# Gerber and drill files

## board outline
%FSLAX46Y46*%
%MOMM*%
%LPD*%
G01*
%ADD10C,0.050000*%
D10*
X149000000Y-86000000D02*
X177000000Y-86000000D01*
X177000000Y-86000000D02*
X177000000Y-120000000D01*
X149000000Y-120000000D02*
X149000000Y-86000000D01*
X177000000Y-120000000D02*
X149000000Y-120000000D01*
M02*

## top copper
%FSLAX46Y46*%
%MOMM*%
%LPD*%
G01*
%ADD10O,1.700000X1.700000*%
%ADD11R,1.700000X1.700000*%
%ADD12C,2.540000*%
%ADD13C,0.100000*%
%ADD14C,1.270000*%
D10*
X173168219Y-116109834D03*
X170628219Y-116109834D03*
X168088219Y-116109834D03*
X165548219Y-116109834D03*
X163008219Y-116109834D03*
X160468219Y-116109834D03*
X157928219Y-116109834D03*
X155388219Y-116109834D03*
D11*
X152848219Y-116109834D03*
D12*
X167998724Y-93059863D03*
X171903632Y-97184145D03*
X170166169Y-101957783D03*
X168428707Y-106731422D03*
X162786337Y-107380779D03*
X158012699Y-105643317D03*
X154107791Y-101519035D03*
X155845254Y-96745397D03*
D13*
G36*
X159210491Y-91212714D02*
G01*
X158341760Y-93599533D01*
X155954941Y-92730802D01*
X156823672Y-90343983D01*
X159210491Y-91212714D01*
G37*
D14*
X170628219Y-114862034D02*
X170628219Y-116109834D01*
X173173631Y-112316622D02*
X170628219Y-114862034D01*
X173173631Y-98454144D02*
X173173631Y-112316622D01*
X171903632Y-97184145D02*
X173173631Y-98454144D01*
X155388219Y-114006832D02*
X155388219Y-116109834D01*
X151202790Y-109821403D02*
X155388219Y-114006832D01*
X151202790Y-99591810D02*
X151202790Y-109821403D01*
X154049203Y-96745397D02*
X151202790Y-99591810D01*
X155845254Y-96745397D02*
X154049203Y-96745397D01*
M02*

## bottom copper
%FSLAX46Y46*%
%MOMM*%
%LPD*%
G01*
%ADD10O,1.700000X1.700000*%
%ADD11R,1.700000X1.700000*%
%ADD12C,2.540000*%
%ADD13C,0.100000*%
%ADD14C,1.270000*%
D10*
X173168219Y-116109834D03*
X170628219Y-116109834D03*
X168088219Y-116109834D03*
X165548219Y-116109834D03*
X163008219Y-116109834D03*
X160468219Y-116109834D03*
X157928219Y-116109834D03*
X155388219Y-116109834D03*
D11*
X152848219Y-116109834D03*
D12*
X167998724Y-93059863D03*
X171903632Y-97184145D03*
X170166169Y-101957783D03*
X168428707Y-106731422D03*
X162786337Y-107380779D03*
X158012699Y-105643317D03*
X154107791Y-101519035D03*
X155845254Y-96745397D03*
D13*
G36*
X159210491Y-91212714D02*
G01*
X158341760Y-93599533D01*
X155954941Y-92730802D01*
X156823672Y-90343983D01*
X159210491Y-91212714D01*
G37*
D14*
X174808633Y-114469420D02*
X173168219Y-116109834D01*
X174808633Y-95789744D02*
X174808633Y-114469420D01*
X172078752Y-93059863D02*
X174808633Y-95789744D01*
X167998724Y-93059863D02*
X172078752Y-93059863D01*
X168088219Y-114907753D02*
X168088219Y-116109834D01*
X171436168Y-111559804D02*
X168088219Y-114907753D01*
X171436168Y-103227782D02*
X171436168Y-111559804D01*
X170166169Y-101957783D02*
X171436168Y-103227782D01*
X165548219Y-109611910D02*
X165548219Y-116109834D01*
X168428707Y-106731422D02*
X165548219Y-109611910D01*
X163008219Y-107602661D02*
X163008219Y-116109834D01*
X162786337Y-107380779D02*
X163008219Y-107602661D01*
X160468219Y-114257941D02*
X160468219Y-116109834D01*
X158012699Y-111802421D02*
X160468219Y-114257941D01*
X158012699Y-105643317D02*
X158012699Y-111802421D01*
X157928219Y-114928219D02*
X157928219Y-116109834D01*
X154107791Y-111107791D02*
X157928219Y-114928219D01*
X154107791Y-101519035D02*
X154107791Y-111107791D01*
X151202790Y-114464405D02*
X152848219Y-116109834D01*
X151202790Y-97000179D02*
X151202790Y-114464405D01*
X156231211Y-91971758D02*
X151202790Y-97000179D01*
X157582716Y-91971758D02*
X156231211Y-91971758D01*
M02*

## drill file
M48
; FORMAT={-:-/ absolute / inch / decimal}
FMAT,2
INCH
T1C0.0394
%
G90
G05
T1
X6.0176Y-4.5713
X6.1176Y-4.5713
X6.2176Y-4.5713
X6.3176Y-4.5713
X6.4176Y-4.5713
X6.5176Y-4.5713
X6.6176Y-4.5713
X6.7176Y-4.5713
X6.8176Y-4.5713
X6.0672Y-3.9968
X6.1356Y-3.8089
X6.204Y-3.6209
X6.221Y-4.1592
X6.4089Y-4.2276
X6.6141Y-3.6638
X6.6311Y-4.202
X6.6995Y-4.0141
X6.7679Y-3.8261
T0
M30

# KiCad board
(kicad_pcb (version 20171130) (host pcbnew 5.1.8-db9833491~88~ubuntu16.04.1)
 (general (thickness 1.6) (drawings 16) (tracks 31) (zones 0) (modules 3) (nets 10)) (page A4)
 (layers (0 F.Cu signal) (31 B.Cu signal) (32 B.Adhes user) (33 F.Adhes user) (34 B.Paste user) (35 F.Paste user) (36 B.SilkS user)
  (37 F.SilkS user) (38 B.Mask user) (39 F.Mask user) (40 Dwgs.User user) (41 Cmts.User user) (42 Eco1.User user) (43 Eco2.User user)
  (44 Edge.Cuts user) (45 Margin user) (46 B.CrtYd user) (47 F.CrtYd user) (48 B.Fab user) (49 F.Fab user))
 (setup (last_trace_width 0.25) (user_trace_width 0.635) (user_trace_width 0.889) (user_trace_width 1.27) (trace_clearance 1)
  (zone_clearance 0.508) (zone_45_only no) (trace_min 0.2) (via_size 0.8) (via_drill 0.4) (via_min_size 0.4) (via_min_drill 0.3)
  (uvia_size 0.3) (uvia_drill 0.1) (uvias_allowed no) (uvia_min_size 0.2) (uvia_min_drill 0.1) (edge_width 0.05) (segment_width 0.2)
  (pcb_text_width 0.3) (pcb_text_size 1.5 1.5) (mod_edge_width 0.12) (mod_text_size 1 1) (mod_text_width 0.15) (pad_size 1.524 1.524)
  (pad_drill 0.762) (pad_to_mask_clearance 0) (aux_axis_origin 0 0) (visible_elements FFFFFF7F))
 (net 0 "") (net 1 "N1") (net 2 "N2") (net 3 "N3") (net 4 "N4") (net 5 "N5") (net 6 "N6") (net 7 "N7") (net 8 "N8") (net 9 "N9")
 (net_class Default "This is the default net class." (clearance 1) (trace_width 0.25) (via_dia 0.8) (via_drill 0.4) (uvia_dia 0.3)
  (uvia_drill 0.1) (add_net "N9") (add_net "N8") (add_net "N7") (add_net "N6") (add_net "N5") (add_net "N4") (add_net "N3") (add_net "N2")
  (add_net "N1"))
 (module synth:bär (layer F.Cu) (at 162.3 98.6)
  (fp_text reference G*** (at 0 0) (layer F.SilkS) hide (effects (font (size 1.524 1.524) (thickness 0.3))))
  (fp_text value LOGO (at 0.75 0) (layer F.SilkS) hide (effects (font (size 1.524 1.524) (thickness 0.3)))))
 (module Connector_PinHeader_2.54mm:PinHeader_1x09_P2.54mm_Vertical (layer F.Cu) (at 152.848219 116.109834 90)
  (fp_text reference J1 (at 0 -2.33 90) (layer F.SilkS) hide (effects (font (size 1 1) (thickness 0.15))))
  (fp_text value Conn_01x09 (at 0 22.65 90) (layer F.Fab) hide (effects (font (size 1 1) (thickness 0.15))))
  (pad 9 thru_hole oval (at 0 20.32 90) (size 1.7 1.7) (drill 1) (layers *.Cu *.Mask) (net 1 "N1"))
  (pad 8 thru_hole oval (at 0 17.78 90) (size 1.7 1.7) (drill 1) (layers *.Cu *.Mask) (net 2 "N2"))
  (pad 7 thru_hole oval (at 0 15.24 90) (size 1.7 1.7) (drill 1) (layers *.Cu *.Mask) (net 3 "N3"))
  (pad 6 thru_hole oval (at 0 12.7 90) (size 1.7 1.7) (drill 1) (layers *.Cu *.Mask) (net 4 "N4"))
  (pad 5 thru_hole oval (at 0 10.16 90) (size 1.7 1.7) (drill 1) (layers *.Cu *.Mask) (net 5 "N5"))
  (pad 4 thru_hole oval (at 0 7.62 90) (size 1.7 1.7) (drill 1) (layers *.Cu *.Mask) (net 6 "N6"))
  (pad 3 thru_hole oval (at 0 5.08 90) (size 1.7 1.7) (drill 1) (layers *.Cu *.Mask) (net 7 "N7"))
  (pad 2 thru_hole oval (at 0 2.54 90) (size 1.7 1.7) (drill 1) (layers *.Cu *.Mask) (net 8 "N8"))
  (pad 1 thru_hole rect (at 0 0 90) (size 1.7 1.7) (drill 1) (layers *.Cu *.Mask) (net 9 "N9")))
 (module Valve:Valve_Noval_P (layer F.Cu) (at 157.582716 91.971758 160)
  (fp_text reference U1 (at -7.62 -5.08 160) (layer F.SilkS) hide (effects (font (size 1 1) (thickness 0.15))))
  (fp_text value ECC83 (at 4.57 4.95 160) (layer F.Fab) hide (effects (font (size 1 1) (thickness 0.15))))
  (pad 9 thru_hole circle (at -10.16 2.54 160) (size 2.54 5.08) (drill 1) (layers *.Cu *.Mask) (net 1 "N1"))
  (pad 8 thru_hole circle (at -15.24 0 160) (size 2.54 5.08) (drill 1) (layers *.Cu *.Mask) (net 2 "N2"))
  (pad 7 thru_hole circle (at -15.24 -5.08 160) (size 2.54 5.08) (drill 1) (layers *.Cu *.Mask) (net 3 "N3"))
  (pad 6 thru_hole circle (at -15.24 -10.16 160) (size 2.54 5.08) (drill 1) (layers *.Cu *.Mask) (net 4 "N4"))
  (pad 5 thru_hole circle (at -10.16 -12.7 160) (size 2.54 5.08) (drill 1) (layers *.Cu *.Mask) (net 5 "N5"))
  (pad 4 thru_hole circle (at -5.08 -12.7 160) (size 2.54 5.08) (drill 1) (layers *.Cu *.Mask) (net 6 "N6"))
  (pad 3 thru_hole circle (at 0 -10.16 160) (size 2.54 5.08) (drill 1) (layers *.Cu *.Mask) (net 7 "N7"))
  (pad 2 thru_hole circle (at 0 -5.08 160) (size 2.54 5.08) (drill 1) (layers *.Cu *.Mask) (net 8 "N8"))
  (pad 1 thru_hole rect (at 0 0 160) (size 2.54 2.54) (drill 1) (layers *.Cu *.Mask) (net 9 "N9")))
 (gr_line (start 149 86) (end 177 86) (layer Edge.Cuts) (width 0.05))
 (gr_line (start 177 86) (end 177 120) (layer Edge.Cuts) (width 0.05))
 (gr_line (start 149 120) (end 149 86) (layer Edge.Cuts) (width 0.05))
 (gr_line (start 177 120) (end 149 120) (layer Edge.Cuts) (width 0.05))
 (segment (start 174.808633 114.46942) (end 173.168219 116.109834) (width 1.27) (layer B.Cu) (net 1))
 (segment (start 174.808633 95.789744) (end 174.808633 114.46942) (width 1.27) (layer B.Cu) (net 1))
 (segment (start 172.078752 93.059863) (end 174.808633 95.789744) (width 1.27) (layer B.Cu) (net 1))
 (segment (start 167.998724 93.059863) (end 172.078752 93.059863) (width 1.27) (layer B.Cu) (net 1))
 (segment (start 170.628219 114.862034) (end 170.628219 116.109834) (width 1.27) (layer F.Cu) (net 2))
 (segment (start 173.173631 112.316622) (end 170.628219 114.862034) (width 1.27) (layer F.Cu) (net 2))
 (segment (start 173.173631 98.454144) (end 173.173631 112.316622) (width 1.27) (layer F.Cu) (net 2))
 (segment (start 171.903632 97.184145) (end 173.173631 98.454144) (width 1.27) (layer F.Cu) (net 2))
 (segment (start 168.088219 114.907753) (end 168.088219 116.109834) (width 1.27) (layer B.Cu) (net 3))
 (segment (start 171.436168 111.559804) (end 168.088219 114.907753) (width 1.27) (layer B.Cu) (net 3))
 (segment (start 171.436168 103.227782) (end 171.436168 111.559804) (width 1.27) (layer B.Cu) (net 3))
 (segment (start 170.166169 101.957783) (end 171.436168 103.227782) (width 1.27) (layer B.Cu) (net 3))
 (segment (start 165.548219 109.61191) (end 165.548219 116.109834) (width 1.27) (layer B.Cu) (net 4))
 (segment (start 168.428707 106.731422) (end 165.548219 109.61191) (width 1.27) (layer B.Cu) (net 4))
 (segment (start 163.008219 107.602661) (end 163.008219 116.109834) (width 1.27) (layer B.Cu) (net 5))
 (segment (start 162.786337 107.380779) (end 163.008219 107.602661) (width 1.27) (layer B.Cu) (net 5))
 (segment (start 160.468219 114.257941) (end 160.468219 116.109834) (width 1.27) (layer B.Cu) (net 6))
 (segment (start 158.012699 111.802421) (end 160.468219 114.257941) (width 1.27) (layer B.Cu) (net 6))
 (segment (start 158.012699 105.643317) (end 158.012699 111.802421) (width 1.27) (layer B.Cu) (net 6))
 (segment (start 157.928219 114.928219) (end 157.928219 116.109834) (width 1.27) (layer B.Cu) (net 7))
 (segment (start 154.107791 111.107791) (end 157.928219 114.928219) (width 1.27) (layer B.Cu) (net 7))
 (segment (start 154.107791 101.519035) (end 154.107791 111.107791) (width 1.27) (layer B.Cu) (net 7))
 (segment (start 155.388219 114.006832) (end 155.388219 116.109834) (width 1.27) (layer F.Cu) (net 8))
 (segment (start 151.20279 109.821403) (end 155.388219 114.006832) (width 1.27) (layer F.Cu) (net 8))
 (segment (start 151.20279 99.59181) (end 151.20279 109.821403) (width 1.27) (layer F.Cu) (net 8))
 (segment (start 154.049203 96.745397) (end 151.20279 99.59181) (width 1.27) (layer F.Cu) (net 8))
 (segment (start 155.845254 96.745397) (end 154.049203 96.745397) (width 1.27) (layer F.Cu) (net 8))
 (segment (start 151.20279 114.464405) (end 152.848219 116.109834) (width 1.27) (layer B.Cu) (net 9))
 (segment (start 151.20279 97.000179) (end 151.20279 114.464405) (width 1.27) (layer B.Cu) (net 9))
 (segment (start 156.231211 91.971758) (end 151.20279 97.000179) (width 1.27) (layer B.Cu) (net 9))
 (segment (start 157.582716 91.971758) (end 156.231211 91.971758) (width 1.27) (layer B.Cu) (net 9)))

